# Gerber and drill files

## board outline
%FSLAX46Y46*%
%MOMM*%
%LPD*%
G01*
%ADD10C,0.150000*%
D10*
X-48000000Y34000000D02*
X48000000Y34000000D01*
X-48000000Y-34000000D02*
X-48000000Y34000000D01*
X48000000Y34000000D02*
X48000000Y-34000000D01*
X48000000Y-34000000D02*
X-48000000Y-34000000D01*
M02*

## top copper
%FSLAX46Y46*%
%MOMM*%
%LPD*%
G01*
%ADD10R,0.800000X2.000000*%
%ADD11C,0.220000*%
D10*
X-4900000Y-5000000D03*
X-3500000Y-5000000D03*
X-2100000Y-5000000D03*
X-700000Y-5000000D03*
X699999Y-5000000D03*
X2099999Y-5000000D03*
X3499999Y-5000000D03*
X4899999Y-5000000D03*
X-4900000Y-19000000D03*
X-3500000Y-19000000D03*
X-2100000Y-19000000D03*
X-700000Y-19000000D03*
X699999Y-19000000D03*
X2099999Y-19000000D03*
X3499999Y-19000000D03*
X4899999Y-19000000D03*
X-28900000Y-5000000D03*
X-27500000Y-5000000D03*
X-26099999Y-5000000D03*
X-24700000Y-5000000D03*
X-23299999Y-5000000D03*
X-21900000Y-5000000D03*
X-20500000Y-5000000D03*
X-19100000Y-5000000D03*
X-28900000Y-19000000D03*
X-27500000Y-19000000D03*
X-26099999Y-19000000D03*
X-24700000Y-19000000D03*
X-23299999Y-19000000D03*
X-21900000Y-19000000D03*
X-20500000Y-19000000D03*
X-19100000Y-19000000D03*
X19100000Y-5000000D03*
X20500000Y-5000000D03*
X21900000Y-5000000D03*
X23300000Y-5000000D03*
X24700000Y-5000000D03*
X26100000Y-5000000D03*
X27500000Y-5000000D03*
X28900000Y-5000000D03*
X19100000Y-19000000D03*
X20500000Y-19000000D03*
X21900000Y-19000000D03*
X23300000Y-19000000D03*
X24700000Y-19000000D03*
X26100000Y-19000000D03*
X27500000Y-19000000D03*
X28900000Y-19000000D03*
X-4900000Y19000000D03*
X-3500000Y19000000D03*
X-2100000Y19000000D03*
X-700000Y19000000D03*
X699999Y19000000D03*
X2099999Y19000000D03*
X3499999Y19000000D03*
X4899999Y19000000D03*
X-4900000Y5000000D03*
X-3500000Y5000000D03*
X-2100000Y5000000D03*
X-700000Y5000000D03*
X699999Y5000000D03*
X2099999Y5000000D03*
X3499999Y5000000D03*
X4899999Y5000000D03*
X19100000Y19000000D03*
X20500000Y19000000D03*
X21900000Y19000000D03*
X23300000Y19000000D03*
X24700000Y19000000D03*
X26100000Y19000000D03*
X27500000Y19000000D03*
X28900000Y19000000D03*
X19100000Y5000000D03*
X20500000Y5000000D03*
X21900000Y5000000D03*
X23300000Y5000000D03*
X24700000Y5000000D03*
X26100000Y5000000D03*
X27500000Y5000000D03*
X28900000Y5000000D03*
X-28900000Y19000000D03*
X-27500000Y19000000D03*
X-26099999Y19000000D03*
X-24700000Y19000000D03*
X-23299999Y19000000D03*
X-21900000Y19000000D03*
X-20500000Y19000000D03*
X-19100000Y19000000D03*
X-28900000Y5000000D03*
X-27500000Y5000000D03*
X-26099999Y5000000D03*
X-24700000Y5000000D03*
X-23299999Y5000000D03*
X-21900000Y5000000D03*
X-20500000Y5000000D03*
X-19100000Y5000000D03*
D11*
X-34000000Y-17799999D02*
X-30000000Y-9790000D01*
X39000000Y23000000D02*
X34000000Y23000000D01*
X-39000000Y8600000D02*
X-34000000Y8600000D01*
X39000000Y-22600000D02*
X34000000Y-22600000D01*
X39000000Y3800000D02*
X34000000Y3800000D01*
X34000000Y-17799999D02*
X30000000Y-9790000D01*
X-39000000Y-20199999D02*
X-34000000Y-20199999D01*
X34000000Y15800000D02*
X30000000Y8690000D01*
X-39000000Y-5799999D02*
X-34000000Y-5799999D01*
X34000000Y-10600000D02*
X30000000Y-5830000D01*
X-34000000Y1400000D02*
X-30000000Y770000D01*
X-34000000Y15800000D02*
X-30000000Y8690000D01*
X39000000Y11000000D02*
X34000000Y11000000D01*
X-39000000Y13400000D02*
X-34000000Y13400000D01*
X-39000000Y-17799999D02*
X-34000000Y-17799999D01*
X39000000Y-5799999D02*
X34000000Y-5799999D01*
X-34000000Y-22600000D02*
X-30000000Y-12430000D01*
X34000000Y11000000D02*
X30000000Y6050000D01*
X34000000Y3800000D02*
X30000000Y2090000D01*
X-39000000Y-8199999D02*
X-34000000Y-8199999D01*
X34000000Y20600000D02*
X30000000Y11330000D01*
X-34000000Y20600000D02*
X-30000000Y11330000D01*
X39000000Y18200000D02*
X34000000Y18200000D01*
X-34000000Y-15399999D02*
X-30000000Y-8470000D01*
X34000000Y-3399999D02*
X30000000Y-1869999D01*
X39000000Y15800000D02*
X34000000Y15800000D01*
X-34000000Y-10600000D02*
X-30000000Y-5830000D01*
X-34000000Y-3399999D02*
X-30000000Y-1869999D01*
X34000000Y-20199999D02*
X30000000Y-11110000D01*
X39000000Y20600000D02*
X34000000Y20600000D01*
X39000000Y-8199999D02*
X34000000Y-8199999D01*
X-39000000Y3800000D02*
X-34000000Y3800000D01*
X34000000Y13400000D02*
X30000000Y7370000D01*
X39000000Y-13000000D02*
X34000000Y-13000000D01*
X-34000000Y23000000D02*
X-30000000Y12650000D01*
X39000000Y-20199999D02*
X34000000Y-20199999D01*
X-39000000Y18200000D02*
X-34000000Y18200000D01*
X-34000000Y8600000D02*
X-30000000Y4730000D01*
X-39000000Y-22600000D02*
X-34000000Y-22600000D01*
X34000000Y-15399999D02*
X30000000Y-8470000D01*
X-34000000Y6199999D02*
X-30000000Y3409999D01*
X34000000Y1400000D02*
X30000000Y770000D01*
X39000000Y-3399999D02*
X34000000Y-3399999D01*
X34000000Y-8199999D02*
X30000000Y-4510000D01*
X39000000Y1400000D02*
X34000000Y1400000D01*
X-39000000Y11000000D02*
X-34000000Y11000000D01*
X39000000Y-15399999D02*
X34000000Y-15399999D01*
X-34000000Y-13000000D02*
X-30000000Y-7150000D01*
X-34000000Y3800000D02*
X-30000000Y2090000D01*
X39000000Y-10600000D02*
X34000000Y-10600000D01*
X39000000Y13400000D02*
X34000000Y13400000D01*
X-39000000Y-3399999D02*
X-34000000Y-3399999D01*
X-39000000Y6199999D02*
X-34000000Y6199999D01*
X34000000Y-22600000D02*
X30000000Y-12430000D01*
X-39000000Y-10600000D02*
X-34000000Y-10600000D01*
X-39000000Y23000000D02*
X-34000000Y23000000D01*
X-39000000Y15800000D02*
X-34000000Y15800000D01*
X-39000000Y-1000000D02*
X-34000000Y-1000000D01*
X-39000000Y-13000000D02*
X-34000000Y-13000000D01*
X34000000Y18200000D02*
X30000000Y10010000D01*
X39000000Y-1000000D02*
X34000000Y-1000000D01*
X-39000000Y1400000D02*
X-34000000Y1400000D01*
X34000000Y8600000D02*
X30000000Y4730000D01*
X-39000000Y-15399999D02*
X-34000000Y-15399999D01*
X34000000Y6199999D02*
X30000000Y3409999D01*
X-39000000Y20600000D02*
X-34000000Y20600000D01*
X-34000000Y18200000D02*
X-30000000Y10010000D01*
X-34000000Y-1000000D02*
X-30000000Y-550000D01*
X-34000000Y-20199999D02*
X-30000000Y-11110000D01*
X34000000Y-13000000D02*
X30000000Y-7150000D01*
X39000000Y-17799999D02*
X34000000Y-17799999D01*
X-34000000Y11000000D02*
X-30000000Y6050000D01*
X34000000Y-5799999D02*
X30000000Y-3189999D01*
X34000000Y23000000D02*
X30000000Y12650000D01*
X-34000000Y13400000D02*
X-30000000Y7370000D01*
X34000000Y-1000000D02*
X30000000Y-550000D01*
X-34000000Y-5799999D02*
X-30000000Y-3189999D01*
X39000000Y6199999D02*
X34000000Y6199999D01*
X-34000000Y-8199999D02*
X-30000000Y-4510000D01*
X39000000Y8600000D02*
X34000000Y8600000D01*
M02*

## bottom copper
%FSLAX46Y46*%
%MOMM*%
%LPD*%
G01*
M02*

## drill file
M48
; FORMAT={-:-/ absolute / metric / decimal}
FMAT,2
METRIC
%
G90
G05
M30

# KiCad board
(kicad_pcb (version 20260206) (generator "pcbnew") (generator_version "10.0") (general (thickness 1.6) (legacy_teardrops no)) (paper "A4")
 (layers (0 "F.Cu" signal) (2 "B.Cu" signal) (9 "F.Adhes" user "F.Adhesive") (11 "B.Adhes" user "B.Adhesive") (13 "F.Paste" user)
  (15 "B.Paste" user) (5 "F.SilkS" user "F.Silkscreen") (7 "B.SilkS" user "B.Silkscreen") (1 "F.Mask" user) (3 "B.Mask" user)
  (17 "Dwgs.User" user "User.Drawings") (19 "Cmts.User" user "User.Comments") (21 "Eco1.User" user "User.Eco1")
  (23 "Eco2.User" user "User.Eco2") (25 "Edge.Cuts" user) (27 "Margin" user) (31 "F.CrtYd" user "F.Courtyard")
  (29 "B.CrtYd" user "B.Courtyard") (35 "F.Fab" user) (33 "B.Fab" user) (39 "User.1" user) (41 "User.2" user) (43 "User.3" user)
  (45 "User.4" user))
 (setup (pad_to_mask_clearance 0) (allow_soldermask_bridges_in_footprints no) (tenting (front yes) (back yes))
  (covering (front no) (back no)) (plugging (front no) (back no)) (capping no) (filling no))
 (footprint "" (layer "F.Cu") (at 0 12)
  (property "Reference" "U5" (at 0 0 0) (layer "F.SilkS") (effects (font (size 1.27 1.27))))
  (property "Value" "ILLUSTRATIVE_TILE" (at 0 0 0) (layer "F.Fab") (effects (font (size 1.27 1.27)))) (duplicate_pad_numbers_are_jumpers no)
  (pad "65" smd rect (at -4.9 -7) (size 0.8 2) (layers "F.Cu") (thermal_bridge_angle 45))
  (pad "66" smd rect (at -3.5 -7) (size 0.8 2) (layers "F.Cu") (thermal_bridge_angle 45))
  (pad "67" smd rect (at -2.1 -7) (size 0.8 2) (layers "F.Cu") (thermal_bridge_angle 45))
  (pad "68" smd rect (at -0.7 -7) (size 0.8 2) (layers "F.Cu") (thermal_bridge_angle 45))
  (pad "69" smd rect (at 0.699999 -7) (size 0.8 2) (layers "F.Cu") (thermal_bridge_angle 45))
  (pad "70" smd rect (at 2.099999 -7) (size 0.8 2) (layers "F.Cu") (thermal_bridge_angle 45))
  (pad "71" smd rect (at 3.499999 -7) (size 0.8 2) (layers "F.Cu") (thermal_bridge_angle 45))
  (pad "72" smd rect (at 4.899999 -7) (size 0.8 2) (layers "F.Cu") (thermal_bridge_angle 45))
  (pad "73" smd rect (at -4.9 7) (size 0.8 2) (layers "F.Cu") (thermal_bridge_angle 45))
  (pad "74" smd rect (at -3.5 7) (size 0.8 2) (layers "F.Cu") (thermal_bridge_angle 45))
  (pad "75" smd rect (at -2.1 7) (size 0.8 2) (layers "F.Cu") (thermal_bridge_angle 45))
  (pad "76" smd rect (at -0.7 7) (size 0.8 2) (layers "F.Cu") (thermal_bridge_angle 45))
  (pad "77" smd rect (at 0.699999 7) (size 0.8 2) (layers "F.Cu") (thermal_bridge_angle 45))
  (pad "78" smd rect (at 2.099999 7) (size 0.8 2) (layers "F.Cu") (thermal_bridge_angle 45))
  (pad "79" smd rect (at 3.499999 7) (size 0.8 2) (layers "F.Cu") (thermal_bridge_angle 45))
  (pad "80" smd rect (at 4.899999 7) (size 0.8 2) (layers "F.Cu") (thermal_bridge_angle 45)))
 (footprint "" (layer "F.Cu") (at -24 12)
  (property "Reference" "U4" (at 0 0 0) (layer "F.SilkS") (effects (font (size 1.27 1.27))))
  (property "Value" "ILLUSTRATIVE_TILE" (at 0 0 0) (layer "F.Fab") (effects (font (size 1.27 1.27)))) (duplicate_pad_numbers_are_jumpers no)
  (pad "49" smd rect (at -4.9 -7) (size 0.8 2) (layers "F.Cu") (thermal_bridge_angle 45))
  (pad "50" smd rect (at -3.5 -7) (size 0.8 2) (layers "F.Cu") (thermal_bridge_angle 45))
  (pad "51" smd rect (at -2.099999 -7) (size 0.8 2) (layers "F.Cu") (thermal_bridge_angle 45))
  (pad "52" smd rect (at -0.7 -7) (size 0.8 2) (layers "F.Cu") (thermal_bridge_angle 45))
  (pad "53" smd rect (at 0.700001 -7) (size 0.8 2) (layers "F.Cu") (thermal_bridge_angle 45))
  (pad "54" smd rect (at 2.1 -7) (size 0.8 2) (layers "F.Cu") (thermal_bridge_angle 45))
  (pad "55" smd rect (at 3.5 -7) (size 0.8 2) (layers "F.Cu") (thermal_bridge_angle 45))
  (pad "56" smd rect (at 4.9 -7) (size 0.8 2) (layers "F.Cu") (thermal_bridge_angle 45))
  (pad "57" smd rect (at -4.9 7) (size 0.8 2) (layers "F.Cu") (thermal_bridge_angle 45))
  (pad "58" smd rect (at -3.5 7) (size 0.8 2) (layers "F.Cu") (thermal_bridge_angle 45))
  (pad "59" smd rect (at -2.099999 7) (size 0.8 2) (layers "F.Cu") (thermal_bridge_angle 45))
  (pad "60" smd rect (at -0.7 7) (size 0.8 2) (layers "F.Cu") (thermal_bridge_angle 45))
  (pad "61" smd rect (at 0.700001 7) (size 0.8 2) (layers "F.Cu") (thermal_bridge_angle 45))
  (pad "62" smd rect (at 2.1 7) (size 0.8 2) (layers "F.Cu") (thermal_bridge_angle 45))
  (pad "63" smd rect (at 3.5 7) (size 0.8 2) (layers "F.Cu") (thermal_bridge_angle 45))
  (pad "64" smd rect (at 4.9 7) (size 0.8 2) (layers "F.Cu") (thermal_bridge_angle 45)))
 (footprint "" (layer "F.Cu") (at 24 12)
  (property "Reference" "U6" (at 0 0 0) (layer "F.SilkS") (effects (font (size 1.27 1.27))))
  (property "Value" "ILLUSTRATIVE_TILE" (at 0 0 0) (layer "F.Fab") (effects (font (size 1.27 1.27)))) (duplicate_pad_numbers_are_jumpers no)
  (pad "81" smd rect (at -4.9 -7) (size 0.8 2) (layers "F.Cu") (thermal_bridge_angle 45))
  (pad "82" smd rect (at -3.5 -7) (size 0.8 2) (layers "F.Cu") (thermal_bridge_angle 45))
  (pad "83" smd rect (at -2.1 -7) (size 0.8 2) (layers "F.Cu") (thermal_bridge_angle 45))
  (pad "84" smd rect (at -0.7 -7) (size 0.8 2) (layers "F.Cu") (thermal_bridge_angle 45))
  (pad "85" smd rect (at 0.7 -7) (size 0.8 2) (layers "F.Cu") (thermal_bridge_angle 45))
  (pad "86" smd rect (at 2.1 -7) (size 0.8 2) (layers "F.Cu") (thermal_bridge_angle 45))
  (pad "87" smd rect (at 3.5 -7) (size 0.8 2) (layers "F.Cu") (thermal_bridge_angle 45))
  (pad "88" smd rect (at 4.9 -7) (size 0.8 2) (layers "F.Cu") (thermal_bridge_angle 45))
  (pad "89" smd rect (at -4.9 7) (size 0.8 2) (layers "F.Cu") (thermal_bridge_angle 45))
  (pad "90" smd rect (at -3.5 7) (size 0.8 2) (layers "F.Cu") (thermal_bridge_angle 45))
  (pad "91" smd rect (at -2.1 7) (size 0.8 2) (layers "F.Cu") (thermal_bridge_angle 45))
  (pad "92" smd rect (at -0.7 7) (size 0.8 2) (layers "F.Cu") (thermal_bridge_angle 45))
  (pad "93" smd rect (at 0.7 7) (size 0.8 2) (layers "F.Cu") (thermal_bridge_angle 45))
  (pad "94" smd rect (at 2.1 7) (size 0.8 2) (layers "F.Cu") (thermal_bridge_angle 45))
  (pad "95" smd rect (at 3.5 7) (size 0.8 2) (layers "F.Cu") (thermal_bridge_angle 45))
  (pad "96" smd rect (at 4.9 7) (size 0.8 2) (layers "F.Cu") (thermal_bridge_angle 45)))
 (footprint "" (layer "F.Cu") (at 0 -12)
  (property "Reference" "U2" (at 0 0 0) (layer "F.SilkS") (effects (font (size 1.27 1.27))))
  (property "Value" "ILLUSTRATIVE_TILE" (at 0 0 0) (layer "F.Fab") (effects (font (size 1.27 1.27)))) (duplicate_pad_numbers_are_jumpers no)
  (pad "17" smd rect (at -4.9 -7) (size 0.8 2) (layers "F.Cu") (thermal_bridge_angle 45))
  (pad "18" smd rect (at -3.5 -7) (size 0.8 2) (layers "F.Cu") (thermal_bridge_angle 45))
  (pad "19" smd rect (at -2.1 -7) (size 0.8 2) (layers "F.Cu") (thermal_bridge_angle 45))
  (pad "20" smd rect (at -0.7 -7) (size 0.8 2) (layers "F.Cu") (thermal_bridge_angle 45))
  (pad "21" smd rect (at 0.699999 -7) (size 0.8 2) (layers "F.Cu") (thermal_bridge_angle 45))
  (pad "22" smd rect (at 2.099999 -7) (size 0.8 2) (layers "F.Cu") (thermal_bridge_angle 45))
  (pad "23" smd rect (at 3.499999 -7) (size 0.8 2) (layers "F.Cu") (thermal_bridge_angle 45))
  (pad "24" smd rect (at 4.899999 -7) (size 0.8 2) (layers "F.Cu") (thermal_bridge_angle 45))
  (pad "25" smd rect (at -4.9 7) (size 0.8 2) (layers "F.Cu") (thermal_bridge_angle 45))
  (pad "26" smd rect (at -3.5 7) (size 0.8 2) (layers "F.Cu") (thermal_bridge_angle 45))
  (pad "27" smd rect (at -2.1 7) (size 0.8 2) (layers "F.Cu") (thermal_bridge_angle 45))
  (pad "28" smd rect (at -0.7 7) (size 0.8 2) (layers "F.Cu") (thermal_bridge_angle 45))
  (pad "29" smd rect (at 0.699999 7) (size 0.8 2) (layers "F.Cu") (thermal_bridge_angle 45))
  (pad "30" smd rect (at 2.099999 7) (size 0.8 2) (layers "F.Cu") (thermal_bridge_angle 45))
  (pad "31" smd rect (at 3.499999 7) (size 0.8 2) (layers "F.Cu") (thermal_bridge_angle 45))
  (pad "32" smd rect (at 4.899999 7) (size 0.8 2) (layers "F.Cu") (thermal_bridge_angle 45)))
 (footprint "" (layer "F.Cu") (at 24 -12)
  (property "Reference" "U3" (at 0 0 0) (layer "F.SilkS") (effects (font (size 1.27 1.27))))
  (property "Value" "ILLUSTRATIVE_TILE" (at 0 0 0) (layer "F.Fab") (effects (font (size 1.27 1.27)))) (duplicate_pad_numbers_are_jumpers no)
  (pad "33" smd rect (at -4.9 -7) (size 0.8 2) (layers "F.Cu") (thermal_bridge_angle 45))
  (pad "34" smd rect (at -3.5 -7) (size 0.8 2) (layers "F.Cu") (thermal_bridge_angle 45))
  (pad "35" smd rect (at -2.1 -7) (size 0.8 2) (layers "F.Cu") (thermal_bridge_angle 45))
  (pad "36" smd rect (at -0.7 -7) (size 0.8 2) (layers "F.Cu") (thermal_bridge_angle 45))
  (pad "37" smd rect (at 0.7 -7) (size 0.8 2) (layers "F.Cu") (thermal_bridge_angle 45))
  (pad "38" smd rect (at 2.1 -7) (size 0.8 2) (layers "F.Cu") (thermal_bridge_angle 45))
  (pad "39" smd rect (at 3.5 -7) (size 0.8 2) (layers "F.Cu") (thermal_bridge_angle 45))
  (pad "40" smd rect (at 4.9 -7) (size 0.8 2) (layers "F.Cu") (thermal_bridge_angle 45))
  (pad "41" smd rect (at -4.9 7) (size 0.8 2) (layers "F.Cu") (thermal_bridge_angle 45))
  (pad "42" smd rect (at -3.5 7) (size 0.8 2) (layers "F.Cu") (thermal_bridge_angle 45))
  (pad "43" smd rect (at -2.1 7) (size 0.8 2) (layers "F.Cu") (thermal_bridge_angle 45))
  (pad "44" smd rect (at -0.7 7) (size 0.8 2) (layers "F.Cu") (thermal_bridge_angle 45))
  (pad "45" smd rect (at 0.7 7) (size 0.8 2) (layers "F.Cu") (thermal_bridge_angle 45))
  (pad "46" smd rect (at 2.1 7) (size 0.8 2) (layers "F.Cu") (thermal_bridge_angle 45))
  (pad "47" smd rect (at 3.5 7) (size 0.8 2) (layers "F.Cu") (thermal_bridge_angle 45))
  (pad "48" smd rect (at 4.9 7) (size 0.8 2) (layers "F.Cu") (thermal_bridge_angle 45)))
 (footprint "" (layer "F.Cu") (at -24 -12)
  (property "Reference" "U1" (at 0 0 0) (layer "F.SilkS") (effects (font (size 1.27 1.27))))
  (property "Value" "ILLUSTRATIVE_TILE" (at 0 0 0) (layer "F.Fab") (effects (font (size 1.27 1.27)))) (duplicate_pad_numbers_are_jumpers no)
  (pad "1" smd rect (at -4.9 -7) (size 0.8 2) (layers "F.Cu") (thermal_bridge_angle 45))
  (pad "2" smd rect (at -3.5 -7) (size 0.8 2) (layers "F.Cu") (thermal_bridge_angle 45))
  (pad "3" smd rect (at -2.099999 -7) (size 0.8 2) (layers "F.Cu") (thermal_bridge_angle 45))
  (pad "4" smd rect (at -0.7 -7) (size 0.8 2) (layers "F.Cu") (thermal_bridge_angle 45))
  (pad "5" smd rect (at 0.700001 -7) (size 0.8 2) (layers "F.Cu") (thermal_bridge_angle 45))
  (pad "6" smd rect (at 2.1 -7) (size 0.8 2) (layers "F.Cu") (thermal_bridge_angle 45))
  (pad "7" smd rect (at 3.5 -7) (size 0.8 2) (layers "F.Cu") (thermal_bridge_angle 45))
  (pad "8" smd rect (at 4.9 -7) (size 0.8 2) (layers "F.Cu") (thermal_bridge_angle 45))
  (pad "9" smd rect (at -4.9 7) (size 0.8 2) (layers "F.Cu") (thermal_bridge_angle 45))
  (pad "10" smd rect (at -3.5 7) (size 0.8 2) (layers "F.Cu") (thermal_bridge_angle 45))
  (pad "11" smd rect (at -2.099999 7) (size 0.8 2) (layers "F.Cu") (thermal_bridge_angle 45))
  (pad "12" smd rect (at -0.7 7) (size 0.8 2) (layers "F.Cu") (thermal_bridge_angle 45))
  (pad "13" smd rect (at 0.700001 7) (size 0.8 2) (layers "F.Cu") (thermal_bridge_angle 45))
  (pad "14" smd rect (at 2.1 7) (size 0.8 2) (layers "F.Cu") (thermal_bridge_angle 45))
  (pad "15" smd rect (at 3.5 7) (size 0.8 2) (layers "F.Cu") (thermal_bridge_angle 45))
  (pad "16" smd rect (at 4.9 7) (size 0.8 2) (layers "F.Cu") (thermal_bridge_angle 45)))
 (gr_line (start -48 -34) (end 48 -34) (stroke (width 0.15) (type default)) (layer "Edge.Cuts"))
 (gr_line (start -48 34) (end -48 -34) (stroke (width 0.15) (type default)) (layer "Edge.Cuts"))
 (gr_line (start 48 -34) (end 48 34) (stroke (width 0.15) (type default)) (layer "Edge.Cuts"))
 (gr_line (start 48 34) (end -48 34) (stroke (width 0.15) (type default)) (layer "Edge.Cuts"))
 (segment (start -34 17.799999) (end -30 9.79) (width 0.22) (layer "F.Cu") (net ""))
 (segment (start 39 -23) (end 34 -23) (width 0.22) (layer "F.Cu") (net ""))
 (segment (start -39 -8.6) (end -34 -8.6) (width 0.22) (layer "F.Cu") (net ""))
 (segment (start 39 22.6) (end 34 22.6) (width 0.22) (layer "F.Cu") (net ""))
 (segment (start 39 -3.8) (end 34 -3.8) (width 0.22) (layer "F.Cu") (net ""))
 (segment (start 34 17.799999) (end 30 9.79) (width 0.22) (layer "F.Cu") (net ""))
 (segment (start -39 20.199999) (end -34 20.199999) (width 0.22) (layer "F.Cu") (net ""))
 (segment (start 34 -15.8) (end 30 -8.69) (width 0.22) (layer "F.Cu") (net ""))
 (segment (start -39 5.799999) (end -34 5.799999) (width 0.22) (layer "F.Cu") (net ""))
 (segment (start 34 10.6) (end 30 5.83) (width 0.22) (layer "F.Cu") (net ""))
 (segment (start -34 -1.4) (end -30 -0.77) (width 0.22) (layer "F.Cu") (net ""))
 (segment (start -34 -15.8) (end -30 -8.69) (width 0.22) (layer "F.Cu") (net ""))
 (segment (start 39 -11) (end 34 -11) (width 0.22) (layer "F.Cu") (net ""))
 (segment (start -39 -13.4) (end -34 -13.4) (width 0.22) (layer "F.Cu") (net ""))
 (segment (start -39 17.799999) (end -34 17.799999) (width 0.22) (layer "F.Cu") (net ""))
 (segment (start 39 5.799999) (end 34 5.799999) (width 0.22) (layer "F.Cu") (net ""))
 (segment (start -34 22.6) (end -30 12.43) (width 0.22) (layer "F.Cu") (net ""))
 (segment (start 34 -11) (end 30 -6.05) (width 0.22) (layer "F.Cu") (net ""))
 (segment (start 34 -3.8) (end 30 -2.09) (width 0.22) (layer "F.Cu") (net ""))
 (segment (start -39 8.199999) (end -34 8.199999) (width 0.22) (layer "F.Cu") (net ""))
 (segment (start 34 -20.6) (end 30 -11.33) (width 0.22) (layer "F.Cu") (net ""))
 (segment (start -34 -20.6) (end -30 -11.33) (width 0.22) (layer "F.Cu") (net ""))
 (segment (start 39 -18.2) (end 34 -18.2) (width 0.22) (layer "F.Cu") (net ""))
 (segment (start -34 15.399999) (end -30 8.47) (width 0.22) (layer "F.Cu") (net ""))
 (segment (start 34 3.399999) (end 30 1.869999) (width 0.22) (layer "F.Cu") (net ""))
 (segment (start 39 -15.8) (end 34 -15.8) (width 0.22) (layer "F.Cu") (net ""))
 (segment (start -34 10.6) (end -30 5.83) (width 0.22) (layer "F.Cu") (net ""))
 (segment (start -34 3.399999) (end -30 1.869999) (width 0.22) (layer "F.Cu") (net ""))
 (segment (start 34 20.199999) (end 30 11.11) (width 0.22) (layer "F.Cu") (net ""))
 (segment (start 39 -20.6) (end 34 -20.6) (width 0.22) (layer "F.Cu") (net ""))
 (segment (start 39 8.199999) (end 34 8.199999) (width 0.22) (layer "F.Cu") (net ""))
 (segment (start -39 -3.8) (end -34 -3.8) (width 0.22) (layer "F.Cu") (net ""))
 (segment (start 34 -13.4) (end 30 -7.37) (width 0.22) (layer "F.Cu") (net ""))
 (segment (start 39 13) (end 34 13) (width 0.22) (layer "F.Cu") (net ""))
 (segment (start -34 -23) (end -30 -12.65) (width 0.22) (layer "F.Cu") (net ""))
 (segment (start 39 20.199999) (end 34 20.199999) (width 0.22) (layer "F.Cu") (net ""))
 (segment (start -39 -18.2) (end -34 -18.2) (width 0.22) (layer "F.Cu") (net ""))
 (segment (start -34 -8.6) (end -30 -4.73) (width 0.22) (layer "F.Cu") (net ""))
 (segment (start -39 22.6) (end -34 22.6) (width 0.22) (layer "F.Cu") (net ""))
 (segment (start 34 15.399999) (end 30 8.47) (width 0.22) (layer "F.Cu") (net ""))
 (segment (start -34 -6.199999) (end -30 -3.409999) (width 0.22) (layer "F.Cu") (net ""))
 (segment (start 34 -1.4) (end 30 -0.77) (width 0.22) (layer "F.Cu") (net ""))
 (segment (start 39 3.399999) (end 34 3.399999) (width 0.22) (layer "F.Cu") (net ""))
 (segment (start 34 8.199999) (end 30 4.51) (width 0.22) (layer "F.Cu") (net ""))
 (segment (start 39 -1.4) (end 34 -1.4) (width 0.22) (layer "F.Cu") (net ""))
 (segment (start -39 -11) (end -34 -11) (width 0.22) (layer "F.Cu") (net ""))
 (segment (start 39 15.399999) (end 34 15.399999) (width 0.22) (layer "F.Cu") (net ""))
 (segment (start -34 13) (end -30 7.15) (width 0.22) (layer "F.Cu") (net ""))
 (segment (start -34 -3.8) (end -30 -2.09) (width 0.22) (layer "F.Cu") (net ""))
 (segment (start 39 10.6) (end 34 10.6) (width 0.22) (layer "F.Cu") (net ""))
 (segment (start 39 -13.4) (end 34 -13.4) (width 0.22) (layer "F.Cu") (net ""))
 (segment (start -39 3.399999) (end -34 3.399999) (width 0.22) (layer "F.Cu") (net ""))
 (segment (start -39 -6.199999) (end -34 -6.199999) (width 0.22) (layer "F.Cu") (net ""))
 (segment (start 34 22.6) (end 30 12.43) (width 0.22) (layer "F.Cu") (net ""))
 (segment (start -39 10.6) (end -34 10.6) (width 0.22) (layer "F.Cu") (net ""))
 (segment (start -39 -23) (end -34 -23) (width 0.22) (layer "F.Cu") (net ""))
 (segment (start -39 -15.8) (end -34 -15.8) (width 0.22) (layer "F.Cu") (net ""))
 (segment (start -39 1) (end -34 1) (width 0.22) (layer "F.Cu") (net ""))
 (segment (start -39 13) (end -34 13) (width 0.22) (layer "F.Cu") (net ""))
 (segment (start 34 -18.2) (end 30 -10.01) (width 0.22) (layer "F.Cu") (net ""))
 (segment (start 39 1) (end 34 1) (width 0.22) (layer "F.Cu") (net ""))
 (segment (start -39 -1.4) (end -34 -1.4) (width 0.22) (layer "F.Cu") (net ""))
 (segment (start 34 -8.6) (end 30 -4.73) (width 0.22) (layer "F.Cu") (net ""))
 (segment (start -39 15.399999) (end -34 15.399999) (width 0.22) (layer "F.Cu") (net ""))
 (segment (start 34 -6.199999) (end 30 -3.409999) (width 0.22) (layer "F.Cu") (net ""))
 (segment (start -39 -20.6) (end -34 -20.6) (width 0.22) (layer "F.Cu") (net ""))
 (segment (start -34 -18.2) (end -30 -10.01) (width 0.22) (layer "F.Cu") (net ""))
 (segment (start -34 1) (end -30 0.55) (width 0.22) (layer "F.Cu") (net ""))
 (segment (start -34 20.199999) (end -30 11.11) (width 0.22) (layer "F.Cu") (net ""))
 (segment (start 34 13) (end 30 7.15) (width 0.22) (layer "F.Cu") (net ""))
 (segment (start 39 17.799999) (end 34 17.799999) (width 0.22) (layer "F.Cu") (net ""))
 (segment (start -34 -11) (end -30 -6.05) (width 0.22) (layer "F.Cu") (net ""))
 (segment (start 34 5.799999) (end 30 3.189999) (width 0.22) (layer "F.Cu") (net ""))
 (segment (start 34 -23) (end 30 -12.65) (width 0.22) (layer "F.Cu") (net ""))
 (segment (start -34 -13.4) (end -30 -7.37) (width 0.22) (layer "F.Cu") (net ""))
 (segment (start 34 1) (end 30 0.55) (width 0.22) (layer "F.Cu") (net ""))
 (segment (start -34 5.799999) (end -30 3.189999) (width 0.22) (layer "F.Cu") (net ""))
 (segment (start 39 -6.199999) (end 34 -6.199999) (width 0.22) (layer "F.Cu") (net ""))
 (segment (start -34 8.199999) (end -30 4.51) (width 0.22) (layer "F.Cu") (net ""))
 (segment (start 39 -8.6) (end 34 -8.6) (width 0.22) (layer "F.Cu") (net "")))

